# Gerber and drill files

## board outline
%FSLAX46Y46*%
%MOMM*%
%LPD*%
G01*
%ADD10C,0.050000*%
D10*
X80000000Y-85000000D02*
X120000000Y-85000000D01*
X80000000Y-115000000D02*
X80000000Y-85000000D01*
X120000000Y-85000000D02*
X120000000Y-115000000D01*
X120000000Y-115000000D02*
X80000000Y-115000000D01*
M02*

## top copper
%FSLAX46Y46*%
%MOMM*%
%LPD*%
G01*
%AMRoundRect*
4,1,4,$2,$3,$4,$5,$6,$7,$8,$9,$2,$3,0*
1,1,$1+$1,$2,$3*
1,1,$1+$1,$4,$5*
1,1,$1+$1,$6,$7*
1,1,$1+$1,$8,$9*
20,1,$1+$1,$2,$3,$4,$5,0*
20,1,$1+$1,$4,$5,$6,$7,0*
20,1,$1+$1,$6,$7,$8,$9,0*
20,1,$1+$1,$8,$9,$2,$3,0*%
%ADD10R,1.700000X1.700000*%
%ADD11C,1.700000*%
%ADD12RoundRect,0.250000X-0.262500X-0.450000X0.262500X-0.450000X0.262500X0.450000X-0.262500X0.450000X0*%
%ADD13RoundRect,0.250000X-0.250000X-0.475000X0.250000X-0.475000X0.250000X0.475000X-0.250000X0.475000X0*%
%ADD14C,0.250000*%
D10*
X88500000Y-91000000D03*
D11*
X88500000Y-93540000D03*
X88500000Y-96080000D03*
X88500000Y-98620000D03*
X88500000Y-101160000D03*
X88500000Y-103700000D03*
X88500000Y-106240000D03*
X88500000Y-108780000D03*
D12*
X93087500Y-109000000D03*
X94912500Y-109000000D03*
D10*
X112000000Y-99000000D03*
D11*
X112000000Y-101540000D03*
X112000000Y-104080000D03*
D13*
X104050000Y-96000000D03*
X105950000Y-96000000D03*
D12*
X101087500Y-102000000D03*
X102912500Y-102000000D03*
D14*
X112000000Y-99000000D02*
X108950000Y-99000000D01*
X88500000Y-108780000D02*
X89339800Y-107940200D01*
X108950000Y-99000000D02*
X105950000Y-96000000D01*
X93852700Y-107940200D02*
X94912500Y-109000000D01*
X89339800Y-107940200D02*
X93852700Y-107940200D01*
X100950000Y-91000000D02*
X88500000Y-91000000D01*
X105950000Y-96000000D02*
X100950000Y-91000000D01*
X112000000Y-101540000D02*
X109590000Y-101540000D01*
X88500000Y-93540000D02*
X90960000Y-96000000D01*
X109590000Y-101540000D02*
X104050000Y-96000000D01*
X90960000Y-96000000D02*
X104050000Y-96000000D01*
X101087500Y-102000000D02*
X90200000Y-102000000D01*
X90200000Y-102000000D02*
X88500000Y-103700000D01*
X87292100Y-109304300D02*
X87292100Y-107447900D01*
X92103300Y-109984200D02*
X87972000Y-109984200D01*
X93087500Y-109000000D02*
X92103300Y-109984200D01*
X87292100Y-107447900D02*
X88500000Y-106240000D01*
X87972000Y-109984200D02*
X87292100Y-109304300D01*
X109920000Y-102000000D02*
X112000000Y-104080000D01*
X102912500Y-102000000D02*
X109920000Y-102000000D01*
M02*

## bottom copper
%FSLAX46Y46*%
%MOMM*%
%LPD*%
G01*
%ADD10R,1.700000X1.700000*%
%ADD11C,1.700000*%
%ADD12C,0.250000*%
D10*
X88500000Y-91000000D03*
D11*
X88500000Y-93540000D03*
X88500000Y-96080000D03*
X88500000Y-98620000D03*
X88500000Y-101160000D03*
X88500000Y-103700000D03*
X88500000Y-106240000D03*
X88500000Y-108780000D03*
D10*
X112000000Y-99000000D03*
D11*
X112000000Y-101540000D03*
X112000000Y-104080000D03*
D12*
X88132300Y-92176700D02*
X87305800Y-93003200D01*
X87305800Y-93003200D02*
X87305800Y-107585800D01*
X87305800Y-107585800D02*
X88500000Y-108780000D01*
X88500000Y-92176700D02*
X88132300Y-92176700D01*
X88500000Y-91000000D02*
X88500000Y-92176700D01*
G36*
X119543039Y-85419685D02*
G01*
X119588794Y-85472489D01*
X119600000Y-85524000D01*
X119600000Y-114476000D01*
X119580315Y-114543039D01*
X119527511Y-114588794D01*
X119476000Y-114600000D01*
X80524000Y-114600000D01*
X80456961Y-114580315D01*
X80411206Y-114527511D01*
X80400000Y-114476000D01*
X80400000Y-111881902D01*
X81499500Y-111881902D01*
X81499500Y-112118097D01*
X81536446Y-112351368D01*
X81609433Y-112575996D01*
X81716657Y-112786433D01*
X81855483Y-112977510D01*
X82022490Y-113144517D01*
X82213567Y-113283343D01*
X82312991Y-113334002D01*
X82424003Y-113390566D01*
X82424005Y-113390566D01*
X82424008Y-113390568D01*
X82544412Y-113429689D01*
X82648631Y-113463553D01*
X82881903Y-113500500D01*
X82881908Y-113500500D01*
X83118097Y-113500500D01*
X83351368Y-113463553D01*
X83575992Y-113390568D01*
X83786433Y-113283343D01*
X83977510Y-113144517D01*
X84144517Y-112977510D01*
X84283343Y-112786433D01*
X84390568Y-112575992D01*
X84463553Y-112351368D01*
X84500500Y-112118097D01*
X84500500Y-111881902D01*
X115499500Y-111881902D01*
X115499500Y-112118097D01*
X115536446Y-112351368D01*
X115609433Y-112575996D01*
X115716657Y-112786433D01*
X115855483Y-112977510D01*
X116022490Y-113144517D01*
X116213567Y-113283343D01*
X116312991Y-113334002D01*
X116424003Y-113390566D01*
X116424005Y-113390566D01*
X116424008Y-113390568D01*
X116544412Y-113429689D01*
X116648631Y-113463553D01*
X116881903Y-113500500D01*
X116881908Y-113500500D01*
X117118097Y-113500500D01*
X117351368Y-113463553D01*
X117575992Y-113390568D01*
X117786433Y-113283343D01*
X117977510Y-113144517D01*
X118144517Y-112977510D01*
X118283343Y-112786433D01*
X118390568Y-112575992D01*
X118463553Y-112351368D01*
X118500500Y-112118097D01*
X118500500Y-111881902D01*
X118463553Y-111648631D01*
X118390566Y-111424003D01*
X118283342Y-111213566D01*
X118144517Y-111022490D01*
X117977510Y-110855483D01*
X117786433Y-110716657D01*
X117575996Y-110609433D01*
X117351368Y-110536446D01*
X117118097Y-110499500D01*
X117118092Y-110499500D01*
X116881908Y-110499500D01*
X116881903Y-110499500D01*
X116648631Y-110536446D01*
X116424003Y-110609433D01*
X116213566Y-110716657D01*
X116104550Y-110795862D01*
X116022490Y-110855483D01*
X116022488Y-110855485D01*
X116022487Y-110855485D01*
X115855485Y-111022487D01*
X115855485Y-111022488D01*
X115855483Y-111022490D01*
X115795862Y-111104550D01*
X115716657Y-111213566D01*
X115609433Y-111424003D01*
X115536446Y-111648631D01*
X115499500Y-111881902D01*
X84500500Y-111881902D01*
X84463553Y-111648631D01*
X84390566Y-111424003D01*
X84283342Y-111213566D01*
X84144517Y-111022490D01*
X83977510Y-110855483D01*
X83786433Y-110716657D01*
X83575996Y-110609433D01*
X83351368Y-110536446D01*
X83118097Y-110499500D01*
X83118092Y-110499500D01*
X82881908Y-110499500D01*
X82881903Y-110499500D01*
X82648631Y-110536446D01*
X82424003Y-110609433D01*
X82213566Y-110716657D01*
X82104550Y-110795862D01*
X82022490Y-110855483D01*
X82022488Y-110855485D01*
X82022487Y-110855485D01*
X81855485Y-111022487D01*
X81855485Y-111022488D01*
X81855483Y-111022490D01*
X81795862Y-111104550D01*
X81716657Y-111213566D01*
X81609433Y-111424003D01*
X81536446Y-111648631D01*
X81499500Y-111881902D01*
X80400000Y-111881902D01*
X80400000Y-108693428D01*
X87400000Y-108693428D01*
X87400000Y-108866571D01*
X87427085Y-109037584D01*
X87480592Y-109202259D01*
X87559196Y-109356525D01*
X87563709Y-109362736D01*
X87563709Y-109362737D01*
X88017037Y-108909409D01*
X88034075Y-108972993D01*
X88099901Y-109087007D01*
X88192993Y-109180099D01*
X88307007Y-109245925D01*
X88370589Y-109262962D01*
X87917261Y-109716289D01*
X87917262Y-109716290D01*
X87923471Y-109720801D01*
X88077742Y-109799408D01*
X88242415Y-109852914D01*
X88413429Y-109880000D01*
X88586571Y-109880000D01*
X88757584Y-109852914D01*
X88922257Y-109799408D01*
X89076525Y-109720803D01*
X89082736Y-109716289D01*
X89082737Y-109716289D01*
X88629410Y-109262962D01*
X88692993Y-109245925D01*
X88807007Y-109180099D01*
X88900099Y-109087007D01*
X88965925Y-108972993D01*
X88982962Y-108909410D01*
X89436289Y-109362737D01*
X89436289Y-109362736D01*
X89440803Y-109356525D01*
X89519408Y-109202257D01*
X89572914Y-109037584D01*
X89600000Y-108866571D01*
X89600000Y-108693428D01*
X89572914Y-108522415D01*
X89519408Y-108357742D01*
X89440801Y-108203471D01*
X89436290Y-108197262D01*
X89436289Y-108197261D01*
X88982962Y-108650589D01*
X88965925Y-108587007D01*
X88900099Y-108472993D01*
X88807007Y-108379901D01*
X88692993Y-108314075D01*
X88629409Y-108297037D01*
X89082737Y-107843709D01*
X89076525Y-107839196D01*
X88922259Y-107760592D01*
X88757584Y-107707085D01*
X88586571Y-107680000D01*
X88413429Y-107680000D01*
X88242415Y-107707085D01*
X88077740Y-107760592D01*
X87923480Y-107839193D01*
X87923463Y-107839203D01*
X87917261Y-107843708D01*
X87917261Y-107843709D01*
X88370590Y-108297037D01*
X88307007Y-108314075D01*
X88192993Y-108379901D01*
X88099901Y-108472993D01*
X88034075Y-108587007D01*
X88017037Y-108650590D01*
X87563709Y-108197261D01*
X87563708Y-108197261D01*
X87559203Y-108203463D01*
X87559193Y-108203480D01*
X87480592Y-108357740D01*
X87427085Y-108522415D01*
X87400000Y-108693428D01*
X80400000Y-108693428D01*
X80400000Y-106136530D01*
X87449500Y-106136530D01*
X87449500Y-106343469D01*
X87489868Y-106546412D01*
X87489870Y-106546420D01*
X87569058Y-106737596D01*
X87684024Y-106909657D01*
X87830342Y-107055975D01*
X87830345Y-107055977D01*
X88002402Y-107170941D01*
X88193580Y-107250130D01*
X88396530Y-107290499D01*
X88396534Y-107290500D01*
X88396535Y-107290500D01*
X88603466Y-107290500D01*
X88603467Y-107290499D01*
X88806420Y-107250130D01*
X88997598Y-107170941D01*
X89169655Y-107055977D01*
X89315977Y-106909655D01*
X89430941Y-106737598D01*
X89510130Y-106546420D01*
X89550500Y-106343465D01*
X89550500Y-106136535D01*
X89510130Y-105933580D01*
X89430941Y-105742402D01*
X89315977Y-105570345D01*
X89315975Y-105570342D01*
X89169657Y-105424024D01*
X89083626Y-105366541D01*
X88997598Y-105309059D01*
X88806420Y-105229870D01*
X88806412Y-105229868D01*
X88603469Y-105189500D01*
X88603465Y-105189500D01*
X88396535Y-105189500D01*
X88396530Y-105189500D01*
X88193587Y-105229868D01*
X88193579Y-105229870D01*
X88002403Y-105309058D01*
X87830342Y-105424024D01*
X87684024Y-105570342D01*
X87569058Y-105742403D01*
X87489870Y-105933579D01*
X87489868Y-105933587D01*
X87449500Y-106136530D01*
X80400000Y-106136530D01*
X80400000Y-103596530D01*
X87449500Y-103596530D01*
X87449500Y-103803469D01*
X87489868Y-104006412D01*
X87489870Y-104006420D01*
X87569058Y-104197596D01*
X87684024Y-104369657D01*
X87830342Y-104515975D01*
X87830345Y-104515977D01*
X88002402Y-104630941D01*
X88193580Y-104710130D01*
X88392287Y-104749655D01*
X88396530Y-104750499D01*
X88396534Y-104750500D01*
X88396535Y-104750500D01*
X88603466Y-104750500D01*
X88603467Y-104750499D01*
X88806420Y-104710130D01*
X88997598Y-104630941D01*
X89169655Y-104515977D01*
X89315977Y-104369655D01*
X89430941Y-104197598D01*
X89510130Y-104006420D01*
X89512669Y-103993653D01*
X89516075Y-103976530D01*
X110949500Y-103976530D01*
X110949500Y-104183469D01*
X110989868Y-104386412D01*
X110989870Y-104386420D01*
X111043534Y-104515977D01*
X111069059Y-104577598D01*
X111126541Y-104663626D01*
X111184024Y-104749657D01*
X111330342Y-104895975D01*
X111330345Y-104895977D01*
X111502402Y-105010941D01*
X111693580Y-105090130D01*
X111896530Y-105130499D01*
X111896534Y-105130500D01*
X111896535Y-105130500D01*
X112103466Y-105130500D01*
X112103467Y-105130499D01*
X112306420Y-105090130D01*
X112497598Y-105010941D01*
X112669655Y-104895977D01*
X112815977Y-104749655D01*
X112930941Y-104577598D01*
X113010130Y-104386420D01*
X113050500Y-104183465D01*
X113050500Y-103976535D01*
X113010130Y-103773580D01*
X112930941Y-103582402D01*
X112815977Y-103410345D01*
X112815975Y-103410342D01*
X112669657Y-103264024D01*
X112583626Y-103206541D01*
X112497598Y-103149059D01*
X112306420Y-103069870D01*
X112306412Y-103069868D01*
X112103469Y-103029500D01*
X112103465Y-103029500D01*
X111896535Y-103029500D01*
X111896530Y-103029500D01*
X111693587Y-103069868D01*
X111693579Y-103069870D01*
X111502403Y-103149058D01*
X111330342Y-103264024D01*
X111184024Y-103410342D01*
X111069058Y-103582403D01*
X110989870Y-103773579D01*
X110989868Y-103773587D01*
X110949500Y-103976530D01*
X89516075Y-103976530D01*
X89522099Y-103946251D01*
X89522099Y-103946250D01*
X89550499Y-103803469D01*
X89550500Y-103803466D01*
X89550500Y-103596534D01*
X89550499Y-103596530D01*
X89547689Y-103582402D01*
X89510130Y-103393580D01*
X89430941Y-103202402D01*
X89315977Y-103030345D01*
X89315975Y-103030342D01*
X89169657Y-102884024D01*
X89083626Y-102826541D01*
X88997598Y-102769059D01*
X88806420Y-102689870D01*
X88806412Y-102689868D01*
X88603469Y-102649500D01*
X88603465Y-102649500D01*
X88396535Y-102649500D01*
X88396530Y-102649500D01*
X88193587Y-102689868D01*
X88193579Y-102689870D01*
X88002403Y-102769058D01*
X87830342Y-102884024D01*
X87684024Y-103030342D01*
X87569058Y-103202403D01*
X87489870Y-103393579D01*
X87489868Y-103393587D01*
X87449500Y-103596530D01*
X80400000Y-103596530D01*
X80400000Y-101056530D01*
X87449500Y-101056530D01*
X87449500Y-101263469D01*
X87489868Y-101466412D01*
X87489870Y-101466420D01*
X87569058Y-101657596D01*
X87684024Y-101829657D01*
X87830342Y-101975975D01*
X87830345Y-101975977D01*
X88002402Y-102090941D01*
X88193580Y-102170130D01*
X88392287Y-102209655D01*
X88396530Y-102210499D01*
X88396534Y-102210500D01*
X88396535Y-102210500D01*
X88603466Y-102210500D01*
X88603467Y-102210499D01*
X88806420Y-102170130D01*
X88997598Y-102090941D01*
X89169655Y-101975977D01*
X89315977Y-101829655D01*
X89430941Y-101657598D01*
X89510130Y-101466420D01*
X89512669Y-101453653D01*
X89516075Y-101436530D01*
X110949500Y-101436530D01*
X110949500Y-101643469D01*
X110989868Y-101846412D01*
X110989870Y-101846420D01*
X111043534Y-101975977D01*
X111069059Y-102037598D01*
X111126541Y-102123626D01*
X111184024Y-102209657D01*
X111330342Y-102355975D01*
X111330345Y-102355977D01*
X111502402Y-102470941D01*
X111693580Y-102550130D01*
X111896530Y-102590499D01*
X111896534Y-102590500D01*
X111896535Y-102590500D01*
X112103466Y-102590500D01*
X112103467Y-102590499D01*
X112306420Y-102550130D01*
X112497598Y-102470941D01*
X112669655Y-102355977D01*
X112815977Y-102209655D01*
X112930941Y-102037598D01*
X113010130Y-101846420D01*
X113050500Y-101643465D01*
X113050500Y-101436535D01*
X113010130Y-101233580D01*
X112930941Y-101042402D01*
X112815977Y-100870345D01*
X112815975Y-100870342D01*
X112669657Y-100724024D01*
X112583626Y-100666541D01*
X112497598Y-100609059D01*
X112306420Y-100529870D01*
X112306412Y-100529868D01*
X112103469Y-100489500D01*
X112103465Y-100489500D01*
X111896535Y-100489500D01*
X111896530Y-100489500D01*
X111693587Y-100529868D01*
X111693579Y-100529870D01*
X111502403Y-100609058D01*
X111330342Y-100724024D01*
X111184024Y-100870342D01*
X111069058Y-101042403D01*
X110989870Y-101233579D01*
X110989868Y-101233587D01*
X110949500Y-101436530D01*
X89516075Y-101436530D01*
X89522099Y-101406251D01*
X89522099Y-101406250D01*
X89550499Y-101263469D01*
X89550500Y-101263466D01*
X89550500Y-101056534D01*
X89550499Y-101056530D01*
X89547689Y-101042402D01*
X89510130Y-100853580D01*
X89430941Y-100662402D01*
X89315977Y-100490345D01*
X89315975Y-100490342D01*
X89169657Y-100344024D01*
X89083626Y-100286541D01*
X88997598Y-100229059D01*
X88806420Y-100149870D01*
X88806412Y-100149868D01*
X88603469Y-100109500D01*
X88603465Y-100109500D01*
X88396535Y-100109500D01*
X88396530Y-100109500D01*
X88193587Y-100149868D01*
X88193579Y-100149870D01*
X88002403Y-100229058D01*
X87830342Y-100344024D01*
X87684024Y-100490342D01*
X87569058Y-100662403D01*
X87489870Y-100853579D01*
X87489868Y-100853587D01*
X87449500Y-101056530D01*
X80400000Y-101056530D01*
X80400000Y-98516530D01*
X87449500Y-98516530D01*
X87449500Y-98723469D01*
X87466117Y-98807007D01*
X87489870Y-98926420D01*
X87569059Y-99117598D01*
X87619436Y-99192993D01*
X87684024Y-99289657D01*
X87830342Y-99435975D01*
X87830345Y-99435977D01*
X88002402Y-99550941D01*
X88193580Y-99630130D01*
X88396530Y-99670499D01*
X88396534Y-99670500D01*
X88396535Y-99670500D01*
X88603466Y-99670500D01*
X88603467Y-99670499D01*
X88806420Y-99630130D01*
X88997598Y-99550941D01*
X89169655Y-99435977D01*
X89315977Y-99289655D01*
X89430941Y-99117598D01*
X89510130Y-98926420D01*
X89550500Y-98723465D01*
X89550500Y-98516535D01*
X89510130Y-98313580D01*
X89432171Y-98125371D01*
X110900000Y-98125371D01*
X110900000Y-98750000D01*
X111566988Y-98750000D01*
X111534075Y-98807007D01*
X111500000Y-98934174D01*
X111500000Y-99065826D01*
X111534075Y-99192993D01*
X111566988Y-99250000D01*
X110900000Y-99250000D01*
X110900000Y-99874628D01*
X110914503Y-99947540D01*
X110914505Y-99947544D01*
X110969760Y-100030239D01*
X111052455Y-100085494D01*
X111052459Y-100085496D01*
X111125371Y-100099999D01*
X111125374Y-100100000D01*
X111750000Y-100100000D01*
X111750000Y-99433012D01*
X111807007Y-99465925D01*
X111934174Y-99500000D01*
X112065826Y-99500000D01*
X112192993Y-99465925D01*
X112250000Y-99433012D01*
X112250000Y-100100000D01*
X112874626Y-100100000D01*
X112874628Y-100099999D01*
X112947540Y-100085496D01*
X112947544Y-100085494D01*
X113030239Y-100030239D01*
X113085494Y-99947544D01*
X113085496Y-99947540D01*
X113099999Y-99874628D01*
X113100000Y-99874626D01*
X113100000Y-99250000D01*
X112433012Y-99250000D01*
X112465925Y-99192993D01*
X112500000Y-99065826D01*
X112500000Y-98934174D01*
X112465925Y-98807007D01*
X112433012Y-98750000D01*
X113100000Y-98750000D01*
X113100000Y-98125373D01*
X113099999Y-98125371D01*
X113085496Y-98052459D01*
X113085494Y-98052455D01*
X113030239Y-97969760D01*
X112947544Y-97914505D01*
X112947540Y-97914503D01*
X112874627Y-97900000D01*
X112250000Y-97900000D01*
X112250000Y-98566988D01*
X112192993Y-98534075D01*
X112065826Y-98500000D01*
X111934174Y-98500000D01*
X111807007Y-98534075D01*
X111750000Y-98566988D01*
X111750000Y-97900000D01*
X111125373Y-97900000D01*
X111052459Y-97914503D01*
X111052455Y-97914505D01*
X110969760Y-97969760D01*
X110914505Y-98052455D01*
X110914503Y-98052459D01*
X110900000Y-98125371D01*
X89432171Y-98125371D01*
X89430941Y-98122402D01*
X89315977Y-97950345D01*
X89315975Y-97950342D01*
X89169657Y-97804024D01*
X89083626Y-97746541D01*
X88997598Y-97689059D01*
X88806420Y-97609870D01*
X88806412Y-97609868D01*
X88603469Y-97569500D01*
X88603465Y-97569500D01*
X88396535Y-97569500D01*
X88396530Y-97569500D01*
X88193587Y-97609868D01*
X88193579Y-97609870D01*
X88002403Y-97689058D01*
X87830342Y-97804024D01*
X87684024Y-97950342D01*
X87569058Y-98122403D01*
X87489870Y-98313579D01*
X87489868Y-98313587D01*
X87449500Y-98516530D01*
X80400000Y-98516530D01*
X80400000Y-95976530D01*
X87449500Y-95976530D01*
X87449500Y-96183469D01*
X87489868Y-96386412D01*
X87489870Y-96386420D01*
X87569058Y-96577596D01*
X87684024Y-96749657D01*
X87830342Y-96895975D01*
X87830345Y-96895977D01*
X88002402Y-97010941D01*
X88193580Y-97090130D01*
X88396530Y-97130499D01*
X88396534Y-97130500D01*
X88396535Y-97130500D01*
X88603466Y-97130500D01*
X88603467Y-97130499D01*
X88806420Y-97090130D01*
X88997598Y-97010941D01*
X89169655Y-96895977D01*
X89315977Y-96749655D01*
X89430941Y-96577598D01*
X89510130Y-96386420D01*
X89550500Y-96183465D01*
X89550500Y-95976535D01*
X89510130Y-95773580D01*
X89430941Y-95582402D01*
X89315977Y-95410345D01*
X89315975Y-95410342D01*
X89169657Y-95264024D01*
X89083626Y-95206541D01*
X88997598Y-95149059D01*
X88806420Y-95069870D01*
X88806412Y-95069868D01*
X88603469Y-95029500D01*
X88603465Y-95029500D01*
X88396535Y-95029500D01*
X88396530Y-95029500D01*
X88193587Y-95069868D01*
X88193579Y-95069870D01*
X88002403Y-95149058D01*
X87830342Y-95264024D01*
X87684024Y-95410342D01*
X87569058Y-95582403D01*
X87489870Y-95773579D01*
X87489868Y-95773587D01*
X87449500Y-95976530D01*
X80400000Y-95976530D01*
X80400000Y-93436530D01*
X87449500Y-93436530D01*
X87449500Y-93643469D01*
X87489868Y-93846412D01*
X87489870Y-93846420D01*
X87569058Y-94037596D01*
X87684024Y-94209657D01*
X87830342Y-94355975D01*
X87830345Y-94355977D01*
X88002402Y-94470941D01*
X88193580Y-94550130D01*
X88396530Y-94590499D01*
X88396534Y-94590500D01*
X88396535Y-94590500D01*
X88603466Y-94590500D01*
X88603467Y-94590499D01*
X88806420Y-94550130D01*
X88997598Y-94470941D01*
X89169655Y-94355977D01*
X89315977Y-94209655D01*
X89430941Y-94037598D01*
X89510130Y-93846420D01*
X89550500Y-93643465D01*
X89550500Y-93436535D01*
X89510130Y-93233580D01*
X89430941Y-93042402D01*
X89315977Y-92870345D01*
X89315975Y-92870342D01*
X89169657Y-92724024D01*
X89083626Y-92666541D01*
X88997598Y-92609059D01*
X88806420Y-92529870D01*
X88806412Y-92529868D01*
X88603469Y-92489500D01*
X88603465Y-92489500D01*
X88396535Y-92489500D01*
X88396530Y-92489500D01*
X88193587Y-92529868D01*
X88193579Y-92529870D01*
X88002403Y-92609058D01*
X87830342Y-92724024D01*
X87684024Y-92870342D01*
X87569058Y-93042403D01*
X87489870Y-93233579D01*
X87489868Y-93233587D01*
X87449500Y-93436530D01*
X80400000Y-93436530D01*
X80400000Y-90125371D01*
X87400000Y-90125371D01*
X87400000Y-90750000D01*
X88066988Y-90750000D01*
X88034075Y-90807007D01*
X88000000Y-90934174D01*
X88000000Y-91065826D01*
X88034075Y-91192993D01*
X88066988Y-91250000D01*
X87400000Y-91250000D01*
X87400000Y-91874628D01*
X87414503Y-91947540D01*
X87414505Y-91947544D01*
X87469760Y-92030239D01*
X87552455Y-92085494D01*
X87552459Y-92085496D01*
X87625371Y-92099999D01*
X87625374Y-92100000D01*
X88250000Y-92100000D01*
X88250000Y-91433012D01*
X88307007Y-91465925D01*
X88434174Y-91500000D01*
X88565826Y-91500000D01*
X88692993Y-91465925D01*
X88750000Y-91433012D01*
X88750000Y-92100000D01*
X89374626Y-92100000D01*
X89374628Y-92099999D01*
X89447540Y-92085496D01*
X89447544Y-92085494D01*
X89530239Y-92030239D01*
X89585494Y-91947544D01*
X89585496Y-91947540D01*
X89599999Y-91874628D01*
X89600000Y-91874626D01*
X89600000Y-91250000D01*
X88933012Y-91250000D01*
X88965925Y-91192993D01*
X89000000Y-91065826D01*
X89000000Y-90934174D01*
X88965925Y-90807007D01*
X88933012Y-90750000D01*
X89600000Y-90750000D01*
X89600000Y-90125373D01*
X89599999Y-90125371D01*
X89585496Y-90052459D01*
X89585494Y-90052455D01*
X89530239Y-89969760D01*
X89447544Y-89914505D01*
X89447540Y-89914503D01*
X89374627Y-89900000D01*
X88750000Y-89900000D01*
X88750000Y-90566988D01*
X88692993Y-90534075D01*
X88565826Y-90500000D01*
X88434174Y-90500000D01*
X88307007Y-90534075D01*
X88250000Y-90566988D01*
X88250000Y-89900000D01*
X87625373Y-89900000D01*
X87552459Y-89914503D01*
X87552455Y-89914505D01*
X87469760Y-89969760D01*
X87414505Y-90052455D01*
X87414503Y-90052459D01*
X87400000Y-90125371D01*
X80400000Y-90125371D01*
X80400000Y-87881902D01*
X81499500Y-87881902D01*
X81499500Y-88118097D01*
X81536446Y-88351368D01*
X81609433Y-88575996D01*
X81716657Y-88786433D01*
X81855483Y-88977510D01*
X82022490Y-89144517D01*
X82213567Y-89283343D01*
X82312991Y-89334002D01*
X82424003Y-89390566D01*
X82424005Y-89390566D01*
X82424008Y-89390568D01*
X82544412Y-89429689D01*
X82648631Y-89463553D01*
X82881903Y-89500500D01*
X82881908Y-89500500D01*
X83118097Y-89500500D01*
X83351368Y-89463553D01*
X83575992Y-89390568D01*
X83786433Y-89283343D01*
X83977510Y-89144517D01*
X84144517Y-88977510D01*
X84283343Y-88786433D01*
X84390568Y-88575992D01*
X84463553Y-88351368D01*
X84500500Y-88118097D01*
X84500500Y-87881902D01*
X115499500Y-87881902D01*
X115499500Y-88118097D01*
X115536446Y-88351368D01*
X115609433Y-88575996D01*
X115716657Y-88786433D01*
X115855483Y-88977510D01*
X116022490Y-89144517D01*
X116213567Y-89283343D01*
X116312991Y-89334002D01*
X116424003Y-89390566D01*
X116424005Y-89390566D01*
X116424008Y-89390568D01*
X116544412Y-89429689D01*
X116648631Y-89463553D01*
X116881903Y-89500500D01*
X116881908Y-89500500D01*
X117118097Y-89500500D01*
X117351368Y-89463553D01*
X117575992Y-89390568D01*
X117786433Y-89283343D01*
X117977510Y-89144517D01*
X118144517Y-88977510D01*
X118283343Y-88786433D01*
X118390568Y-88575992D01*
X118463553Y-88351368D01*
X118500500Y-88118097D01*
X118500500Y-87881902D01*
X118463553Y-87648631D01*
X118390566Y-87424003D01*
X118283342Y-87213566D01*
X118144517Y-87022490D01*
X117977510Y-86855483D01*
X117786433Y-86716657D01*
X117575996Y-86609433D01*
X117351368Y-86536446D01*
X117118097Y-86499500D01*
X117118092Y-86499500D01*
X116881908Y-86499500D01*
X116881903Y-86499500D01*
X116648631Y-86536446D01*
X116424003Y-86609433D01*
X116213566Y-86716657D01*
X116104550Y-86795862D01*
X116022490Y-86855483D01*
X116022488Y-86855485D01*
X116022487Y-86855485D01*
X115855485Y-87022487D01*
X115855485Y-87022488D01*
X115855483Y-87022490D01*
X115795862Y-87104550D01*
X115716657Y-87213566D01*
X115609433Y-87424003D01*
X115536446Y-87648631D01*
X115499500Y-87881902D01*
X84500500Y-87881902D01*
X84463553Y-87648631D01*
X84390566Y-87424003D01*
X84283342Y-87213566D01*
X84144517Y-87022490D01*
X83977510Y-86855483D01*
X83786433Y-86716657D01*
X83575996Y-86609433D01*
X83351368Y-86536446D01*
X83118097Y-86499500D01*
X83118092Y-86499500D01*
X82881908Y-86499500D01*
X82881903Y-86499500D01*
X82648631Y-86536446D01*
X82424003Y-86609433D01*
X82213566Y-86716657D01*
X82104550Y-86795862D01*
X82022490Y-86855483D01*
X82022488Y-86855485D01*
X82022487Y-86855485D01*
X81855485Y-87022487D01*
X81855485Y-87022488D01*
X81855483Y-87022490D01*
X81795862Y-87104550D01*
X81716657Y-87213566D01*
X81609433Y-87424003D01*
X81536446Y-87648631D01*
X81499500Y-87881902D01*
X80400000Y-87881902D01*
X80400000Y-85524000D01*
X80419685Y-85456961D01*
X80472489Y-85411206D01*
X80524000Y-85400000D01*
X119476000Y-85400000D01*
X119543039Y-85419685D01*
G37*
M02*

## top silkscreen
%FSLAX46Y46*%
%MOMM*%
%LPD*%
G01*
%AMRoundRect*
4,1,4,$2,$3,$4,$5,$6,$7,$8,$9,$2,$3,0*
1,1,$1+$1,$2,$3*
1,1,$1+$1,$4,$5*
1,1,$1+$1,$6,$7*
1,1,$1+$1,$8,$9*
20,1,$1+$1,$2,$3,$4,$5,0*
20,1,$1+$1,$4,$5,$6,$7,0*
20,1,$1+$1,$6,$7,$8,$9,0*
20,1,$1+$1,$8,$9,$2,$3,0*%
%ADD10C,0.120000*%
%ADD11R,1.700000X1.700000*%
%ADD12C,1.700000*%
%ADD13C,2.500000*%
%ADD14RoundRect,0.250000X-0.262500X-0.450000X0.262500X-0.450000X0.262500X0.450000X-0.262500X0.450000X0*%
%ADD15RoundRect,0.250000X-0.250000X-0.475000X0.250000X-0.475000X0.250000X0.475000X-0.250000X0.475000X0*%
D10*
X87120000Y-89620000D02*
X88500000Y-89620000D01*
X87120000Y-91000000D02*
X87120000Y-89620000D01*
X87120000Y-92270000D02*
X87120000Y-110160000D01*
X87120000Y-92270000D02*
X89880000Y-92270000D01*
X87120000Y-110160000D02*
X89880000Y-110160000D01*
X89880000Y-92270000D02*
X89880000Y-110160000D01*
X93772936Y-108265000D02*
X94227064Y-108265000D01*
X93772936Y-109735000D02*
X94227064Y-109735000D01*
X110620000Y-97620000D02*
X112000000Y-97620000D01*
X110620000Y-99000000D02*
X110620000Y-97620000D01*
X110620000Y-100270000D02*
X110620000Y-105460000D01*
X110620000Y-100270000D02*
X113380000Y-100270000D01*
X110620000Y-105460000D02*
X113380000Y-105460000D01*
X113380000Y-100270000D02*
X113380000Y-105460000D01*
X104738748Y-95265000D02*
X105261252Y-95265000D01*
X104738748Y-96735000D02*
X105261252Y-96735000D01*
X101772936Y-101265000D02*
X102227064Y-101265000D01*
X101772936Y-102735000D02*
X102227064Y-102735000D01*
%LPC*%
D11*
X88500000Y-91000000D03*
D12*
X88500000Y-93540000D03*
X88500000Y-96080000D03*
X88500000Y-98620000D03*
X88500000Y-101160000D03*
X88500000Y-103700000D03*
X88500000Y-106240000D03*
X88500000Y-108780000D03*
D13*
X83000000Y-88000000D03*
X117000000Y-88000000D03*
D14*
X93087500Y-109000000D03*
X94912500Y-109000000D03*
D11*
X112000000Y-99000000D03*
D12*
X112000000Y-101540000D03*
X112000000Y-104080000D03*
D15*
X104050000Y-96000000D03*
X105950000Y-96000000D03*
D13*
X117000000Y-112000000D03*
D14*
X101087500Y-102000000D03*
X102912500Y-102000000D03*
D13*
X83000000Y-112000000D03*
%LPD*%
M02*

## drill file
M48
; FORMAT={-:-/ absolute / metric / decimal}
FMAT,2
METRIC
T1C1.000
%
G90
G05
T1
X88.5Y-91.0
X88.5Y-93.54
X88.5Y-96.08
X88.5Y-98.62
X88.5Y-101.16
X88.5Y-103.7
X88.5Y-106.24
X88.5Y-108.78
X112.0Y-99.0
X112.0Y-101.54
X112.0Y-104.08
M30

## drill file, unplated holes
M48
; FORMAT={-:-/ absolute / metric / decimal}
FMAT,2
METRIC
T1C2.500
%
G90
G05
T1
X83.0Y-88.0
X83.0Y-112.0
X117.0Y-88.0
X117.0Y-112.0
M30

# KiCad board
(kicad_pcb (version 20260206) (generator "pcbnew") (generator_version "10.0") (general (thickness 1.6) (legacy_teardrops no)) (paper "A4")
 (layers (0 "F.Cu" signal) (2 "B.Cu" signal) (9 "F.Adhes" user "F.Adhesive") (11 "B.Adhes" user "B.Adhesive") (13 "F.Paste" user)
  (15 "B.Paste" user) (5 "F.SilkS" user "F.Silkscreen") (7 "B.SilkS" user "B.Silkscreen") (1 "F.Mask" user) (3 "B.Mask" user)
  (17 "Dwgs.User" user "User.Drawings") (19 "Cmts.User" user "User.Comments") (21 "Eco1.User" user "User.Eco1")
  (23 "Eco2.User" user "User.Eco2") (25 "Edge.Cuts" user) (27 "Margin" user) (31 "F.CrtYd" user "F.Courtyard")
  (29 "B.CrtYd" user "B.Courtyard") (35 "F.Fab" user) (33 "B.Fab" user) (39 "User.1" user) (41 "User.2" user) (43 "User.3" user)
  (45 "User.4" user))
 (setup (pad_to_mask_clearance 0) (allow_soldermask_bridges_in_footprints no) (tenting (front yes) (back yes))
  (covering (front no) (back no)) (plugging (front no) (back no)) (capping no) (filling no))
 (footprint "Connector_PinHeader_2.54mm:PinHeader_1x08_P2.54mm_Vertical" (layer "F.Cu") (at 88.5 91)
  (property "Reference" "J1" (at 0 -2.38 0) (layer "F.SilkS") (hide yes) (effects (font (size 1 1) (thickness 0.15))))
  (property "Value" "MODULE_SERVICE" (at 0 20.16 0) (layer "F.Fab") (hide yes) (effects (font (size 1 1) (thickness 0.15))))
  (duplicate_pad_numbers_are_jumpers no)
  (fp_line (start -1.38 -1.38) (end 0 -1.38) (stroke (width 0.12) (type solid)) (layer "F.SilkS"))
  (fp_line (start -1.38 0) (end -1.38 -1.38) (stroke (width 0.12) (type solid)) (layer "F.SilkS"))
  (fp_line (start -1.38 1.27) (end -1.38 19.16) (stroke (width 0.12) (type solid)) (layer "F.SilkS"))
  (fp_line (start -1.38 1.27) (end 1.38 1.27) (stroke (width 0.12) (type solid)) (layer "F.SilkS"))
  (fp_line (start -1.38 19.16) (end 1.38 19.16) (stroke (width 0.12) (type solid)) (layer "F.SilkS"))
  (fp_line (start 1.38 1.27) (end 1.38 19.16) (stroke (width 0.12) (type solid)) (layer "F.SilkS"))
  (pad "1" thru_hole rect (at 0 0) (size 1.7 1.7) (drill 1) (layers "*.Cu" "*.Mask") (remove_unused_layers no) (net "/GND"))
  (pad "2" thru_hole circle (at 0 2.54) (size 1.7 1.7) (drill 1) (layers "*.Cu" "*.Mask") (remove_unused_layers no) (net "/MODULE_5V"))
  (pad "3" thru_hole circle (at 0 5.08) (size 1.7 1.7) (drill 1) (layers "*.Cu" "*.Mask") (remove_unused_layers no)
   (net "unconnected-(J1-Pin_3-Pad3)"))
  (pad "4" thru_hole circle (at 0 7.62) (size 1.7 1.7) (drill 1) (layers "*.Cu" "*.Mask") (remove_unused_layers no)
   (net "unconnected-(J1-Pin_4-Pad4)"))
  (pad "5" thru_hole circle (at 0 10.16) (size 1.7 1.7) (drill 1) (layers "*.Cu" "*.Mask") (remove_unused_layers no)
   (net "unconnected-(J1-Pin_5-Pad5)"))
  (pad "6" thru_hole circle (at 0 12.7) (size 1.7 1.7) (drill 1) (layers "*.Cu" "*.Mask") (remove_unused_layers no) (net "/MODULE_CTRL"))
  (pad "7" thru_hole circle (at 0 15.24) (size 1.7 1.7) (drill 1) (layers "*.Cu" "*.Mask") (remove_unused_layers no) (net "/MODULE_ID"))
  (pad "8" thru_hole circle (at 0 17.78) (size 1.7 1.7) (drill 1) (layers "*.Cu" "*.Mask") (remove_unused_layers no) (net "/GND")))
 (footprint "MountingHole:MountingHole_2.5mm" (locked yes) (layer "F.Cu") (at 83 88)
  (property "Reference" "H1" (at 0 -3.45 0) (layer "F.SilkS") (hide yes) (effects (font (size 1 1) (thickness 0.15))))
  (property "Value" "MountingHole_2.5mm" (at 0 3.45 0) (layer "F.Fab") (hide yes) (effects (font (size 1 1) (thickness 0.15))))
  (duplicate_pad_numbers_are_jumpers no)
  (pad "" np_thru_hole circle (at 0 0) (size 2.5 2.5) (drill 2.5) (layers "*.Cu" "*.Mask")))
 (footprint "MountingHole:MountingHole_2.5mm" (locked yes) (layer "F.Cu") (at 117 88)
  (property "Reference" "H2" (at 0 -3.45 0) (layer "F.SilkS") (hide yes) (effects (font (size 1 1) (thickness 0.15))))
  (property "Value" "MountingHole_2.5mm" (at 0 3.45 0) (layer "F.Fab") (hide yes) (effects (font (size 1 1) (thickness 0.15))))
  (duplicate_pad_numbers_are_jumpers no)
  (pad "" np_thru_hole circle (at 0 0) (size 2.5 2.5) (drill 2.5) (layers "*.Cu" "*.Mask")))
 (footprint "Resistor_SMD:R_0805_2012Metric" (layer "F.Cu") (at 94 109)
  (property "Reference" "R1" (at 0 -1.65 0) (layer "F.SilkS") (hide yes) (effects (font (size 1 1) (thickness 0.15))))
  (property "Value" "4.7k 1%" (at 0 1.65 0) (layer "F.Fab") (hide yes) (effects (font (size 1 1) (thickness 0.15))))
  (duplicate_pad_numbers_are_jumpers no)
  (fp_line (start -0.227064 -0.735) (end 0.227064 -0.735) (stroke (width 0.12) (type solid)) (layer "F.SilkS"))
  (fp_line (start -0.227064 0.735) (end 0.227064 0.735) (stroke (width 0.12) (type solid)) (layer "F.SilkS"))
  (pad "1" smd roundrect (at -0.9125 0) (size 1.025 1.4) (layers "F.Cu" "F.Mask" "F.Paste") (roundrect_rratio 0.243902) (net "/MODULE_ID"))
  (pad "2" smd roundrect (at 0.9125 0) (size 1.025 1.4) (layers "F.Cu" "F.Mask" "F.Paste") (roundrect_rratio 0.243902) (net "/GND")))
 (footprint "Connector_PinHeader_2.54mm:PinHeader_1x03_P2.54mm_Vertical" (layer "F.Cu") (at 112 99)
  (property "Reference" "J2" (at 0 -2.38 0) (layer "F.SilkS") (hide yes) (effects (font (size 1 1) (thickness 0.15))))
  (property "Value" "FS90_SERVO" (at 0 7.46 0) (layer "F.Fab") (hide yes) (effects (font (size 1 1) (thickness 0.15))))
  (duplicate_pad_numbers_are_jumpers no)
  (fp_line (start -1.38 -1.38) (end 0 -1.38) (stroke (width 0.12) (type solid)) (layer "F.SilkS"))
  (fp_line (start -1.38 0) (end -1.38 -1.38) (stroke (width 0.12) (type solid)) (layer "F.SilkS"))
  (fp_line (start -1.38 1.27) (end -1.38 6.46) (stroke (width 0.12) (type solid)) (layer "F.SilkS"))
  (fp_line (start -1.38 1.27) (end 1.38 1.27) (stroke (width 0.12) (type solid)) (layer "F.SilkS"))
  (fp_line (start -1.38 6.46) (end 1.38 6.46) (stroke (width 0.12) (type solid)) (layer "F.SilkS"))
  (fp_line (start 1.38 1.27) (end 1.38 6.46) (stroke (width 0.12) (type solid)) (layer "F.SilkS"))
  (pad "1" thru_hole rect (at 0 0) (size 1.7 1.7) (drill 1) (layers "*.Cu" "*.Mask") (remove_unused_layers no) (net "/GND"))
  (pad "2" thru_hole circle (at 0 2.54) (size 1.7 1.7) (drill 1) (layers "*.Cu" "*.Mask") (remove_unused_layers no) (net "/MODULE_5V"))
  (pad "3" thru_hole circle (at 0 5.08) (size 1.7 1.7) (drill 1) (layers "*.Cu" "*.Mask") (remove_unused_layers no) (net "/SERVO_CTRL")))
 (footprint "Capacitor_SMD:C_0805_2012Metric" (layer "F.Cu") (at 105 96)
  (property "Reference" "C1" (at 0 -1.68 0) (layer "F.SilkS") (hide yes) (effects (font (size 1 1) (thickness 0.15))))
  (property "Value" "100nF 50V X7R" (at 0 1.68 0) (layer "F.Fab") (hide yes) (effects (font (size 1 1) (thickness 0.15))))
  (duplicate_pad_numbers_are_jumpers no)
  (fp_line (start -0.261252 -0.735) (end 0.261252 -0.735) (stroke (width 0.12) (type solid)) (layer "F.SilkS"))
  (fp_line (start -0.261252 0.735) (end 0.261252 0.735) (stroke (width 0.12) (type solid)) (layer "F.SilkS"))
  (pad "1" smd roundrect (at -0.95 0) (size 1 1.45) (layers "F.Cu" "F.Mask" "F.Paste") (roundrect_rratio 0.25) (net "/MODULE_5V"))
  (pad "2" smd roundrect (at 0.95 0) (size 1 1.45) (layers "F.Cu" "F.Mask" "F.Paste") (roundrect_rratio 0.25) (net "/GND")))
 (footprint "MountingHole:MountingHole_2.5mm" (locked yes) (layer "F.Cu") (at 117 112)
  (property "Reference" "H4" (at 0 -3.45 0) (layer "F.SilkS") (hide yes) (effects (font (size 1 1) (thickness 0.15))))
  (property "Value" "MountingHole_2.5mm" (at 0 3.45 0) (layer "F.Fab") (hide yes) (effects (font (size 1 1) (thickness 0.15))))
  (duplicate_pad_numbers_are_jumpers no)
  (pad "" np_thru_hole circle (at 0 0) (size 2.5 2.5) (drill 2.5) (layers "*.Cu" "*.Mask")))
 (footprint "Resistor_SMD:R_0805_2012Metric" (layer "F.Cu") (at 102 102)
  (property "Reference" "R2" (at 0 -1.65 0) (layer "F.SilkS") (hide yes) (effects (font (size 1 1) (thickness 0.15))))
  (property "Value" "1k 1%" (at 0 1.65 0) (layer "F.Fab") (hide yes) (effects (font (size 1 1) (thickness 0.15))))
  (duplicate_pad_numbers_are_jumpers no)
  (fp_line (start -0.227064 -0.735) (end 0.227064 -0.735) (stroke (width 0.12) (type solid)) (layer "F.SilkS"))
  (fp_line (start -0.227064 0.735) (end 0.227064 0.735) (stroke (width 0.12) (type solid)) (layer "F.SilkS"))
  (pad "1" smd roundrect (at -0.9125 0) (size 1.025 1.4) (layers "F.Cu" "F.Mask" "F.Paste") (roundrect_rratio 0.243902) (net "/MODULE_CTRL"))
  (pad "2" smd roundrect (at 0.9125 0) (size 1.025 1.4) (layers "F.Cu" "F.Mask" "F.Paste") (roundrect_rratio 0.243902) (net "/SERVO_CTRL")))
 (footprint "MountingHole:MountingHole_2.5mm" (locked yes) (layer "F.Cu") (at 83 112)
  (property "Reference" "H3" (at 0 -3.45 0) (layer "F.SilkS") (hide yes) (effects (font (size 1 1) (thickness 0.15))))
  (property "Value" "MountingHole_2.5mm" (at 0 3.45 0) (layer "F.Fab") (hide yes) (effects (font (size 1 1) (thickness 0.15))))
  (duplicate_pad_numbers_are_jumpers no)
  (pad "" np_thru_hole circle (at 0 0) (size 2.5 2.5) (drill 2.5) (layers "*.Cu" "*.Mask")))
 (gr_line (start 80 85) (end 120 85) (stroke (width 0.05) (type default)) (layer "Edge.Cuts"))
 (gr_line (start 80 115) (end 80 85) (stroke (width 0.05) (type default)) (layer "Edge.Cuts"))
 (gr_line (start 120 85) (end 120 115) (stroke (width 0.05) (type default)) (layer "Edge.Cuts"))
 (gr_line (start 120 115) (end 80 115) (stroke (width 0.05) (type default)) (layer "Edge.Cuts"))
 (segment (start 112 99) (end 108.95 99) (width 0.25) (layer "F.Cu") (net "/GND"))
 (segment (start 88.5 108.78) (end 89.3398 107.9402) (width 0.25) (layer "F.Cu") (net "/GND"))
 (segment (start 108.95 99) (end 105.95 96) (width 0.25) (layer "F.Cu") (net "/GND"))
 (segment (start 93.8527 107.9402) (end 94.9125 109) (width 0.25) (layer "F.Cu") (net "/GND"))
 (segment (start 89.3398 107.9402) (end 93.8527 107.9402) (width 0.25) (layer "F.Cu") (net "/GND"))
 (segment (start 100.95 91) (end 88.5 91) (width 0.25) (layer "F.Cu") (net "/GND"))
 (segment (start 105.95 96) (end 100.95 91) (width 0.25) (layer "F.Cu") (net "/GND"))
 (segment (start 88.1323 92.1767) (end 87.3058 93.0032) (width 0.25) (layer "B.Cu") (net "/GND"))
 (segment (start 87.3058 93.0032) (end 87.3058 107.5858) (width 0.25) (layer "B.Cu") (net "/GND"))
 (segment (start 87.3058 107.5858) (end 88.5 108.78) (width 0.25) (layer "B.Cu") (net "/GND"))
 (segment (start 88.5 92.1767) (end 88.1323 92.1767) (width 0.25) (layer "B.Cu") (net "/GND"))
 (segment (start 88.5 91) (end 88.5 92.1767) (width 0.25) (layer "B.Cu") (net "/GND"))
 (segment (start 112 101.54) (end 109.59 101.54) (width 0.25) (layer "F.Cu") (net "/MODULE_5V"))
 (segment (start 88.5 93.54) (end 90.96 96) (width 0.25) (layer "F.Cu") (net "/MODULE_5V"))
 (segment (start 109.59 101.54) (end 104.05 96) (width 0.25) (layer "F.Cu") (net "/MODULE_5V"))
 (segment (start 90.96 96) (end 104.05 96) (width 0.25) (layer "F.Cu") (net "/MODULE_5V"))
 (segment (start 101.0875 102) (end 90.2 102) (width 0.25) (layer "F.Cu") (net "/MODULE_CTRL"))
 (segment (start 90.2 102) (end 88.5 103.7) (width 0.25) (layer "F.Cu") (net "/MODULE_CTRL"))
 (segment (start 87.2921 109.3043) (end 87.2921 107.4479) (width 0.25) (layer "F.Cu") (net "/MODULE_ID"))
 (segment (start 92.1033 109.9842) (end 87.972 109.9842) (width 0.25) (layer "F.Cu") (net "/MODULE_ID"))
 (segment (start 93.0875 109) (end 92.1033 109.9842) (width 0.25) (layer "F.Cu") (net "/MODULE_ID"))
 (segment (start 87.2921 107.4479) (end 88.5 106.24) (width 0.25) (layer "F.Cu") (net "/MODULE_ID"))
 (segment (start 87.972 109.9842) (end 87.2921 109.3043) (width 0.25) (layer "F.Cu") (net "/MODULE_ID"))
 (segment (start 109.92 102) (end 112 104.08) (width 0.25) (layer "F.Cu") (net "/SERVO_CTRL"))
 (segment (start 102.9125 102) (end 109.92 102) (width 0.25) (layer "F.Cu") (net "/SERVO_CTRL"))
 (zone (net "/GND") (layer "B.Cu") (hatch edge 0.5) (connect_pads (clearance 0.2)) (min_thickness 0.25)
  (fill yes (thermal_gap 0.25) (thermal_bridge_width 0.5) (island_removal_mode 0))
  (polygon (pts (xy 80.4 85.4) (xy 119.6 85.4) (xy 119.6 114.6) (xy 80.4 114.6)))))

